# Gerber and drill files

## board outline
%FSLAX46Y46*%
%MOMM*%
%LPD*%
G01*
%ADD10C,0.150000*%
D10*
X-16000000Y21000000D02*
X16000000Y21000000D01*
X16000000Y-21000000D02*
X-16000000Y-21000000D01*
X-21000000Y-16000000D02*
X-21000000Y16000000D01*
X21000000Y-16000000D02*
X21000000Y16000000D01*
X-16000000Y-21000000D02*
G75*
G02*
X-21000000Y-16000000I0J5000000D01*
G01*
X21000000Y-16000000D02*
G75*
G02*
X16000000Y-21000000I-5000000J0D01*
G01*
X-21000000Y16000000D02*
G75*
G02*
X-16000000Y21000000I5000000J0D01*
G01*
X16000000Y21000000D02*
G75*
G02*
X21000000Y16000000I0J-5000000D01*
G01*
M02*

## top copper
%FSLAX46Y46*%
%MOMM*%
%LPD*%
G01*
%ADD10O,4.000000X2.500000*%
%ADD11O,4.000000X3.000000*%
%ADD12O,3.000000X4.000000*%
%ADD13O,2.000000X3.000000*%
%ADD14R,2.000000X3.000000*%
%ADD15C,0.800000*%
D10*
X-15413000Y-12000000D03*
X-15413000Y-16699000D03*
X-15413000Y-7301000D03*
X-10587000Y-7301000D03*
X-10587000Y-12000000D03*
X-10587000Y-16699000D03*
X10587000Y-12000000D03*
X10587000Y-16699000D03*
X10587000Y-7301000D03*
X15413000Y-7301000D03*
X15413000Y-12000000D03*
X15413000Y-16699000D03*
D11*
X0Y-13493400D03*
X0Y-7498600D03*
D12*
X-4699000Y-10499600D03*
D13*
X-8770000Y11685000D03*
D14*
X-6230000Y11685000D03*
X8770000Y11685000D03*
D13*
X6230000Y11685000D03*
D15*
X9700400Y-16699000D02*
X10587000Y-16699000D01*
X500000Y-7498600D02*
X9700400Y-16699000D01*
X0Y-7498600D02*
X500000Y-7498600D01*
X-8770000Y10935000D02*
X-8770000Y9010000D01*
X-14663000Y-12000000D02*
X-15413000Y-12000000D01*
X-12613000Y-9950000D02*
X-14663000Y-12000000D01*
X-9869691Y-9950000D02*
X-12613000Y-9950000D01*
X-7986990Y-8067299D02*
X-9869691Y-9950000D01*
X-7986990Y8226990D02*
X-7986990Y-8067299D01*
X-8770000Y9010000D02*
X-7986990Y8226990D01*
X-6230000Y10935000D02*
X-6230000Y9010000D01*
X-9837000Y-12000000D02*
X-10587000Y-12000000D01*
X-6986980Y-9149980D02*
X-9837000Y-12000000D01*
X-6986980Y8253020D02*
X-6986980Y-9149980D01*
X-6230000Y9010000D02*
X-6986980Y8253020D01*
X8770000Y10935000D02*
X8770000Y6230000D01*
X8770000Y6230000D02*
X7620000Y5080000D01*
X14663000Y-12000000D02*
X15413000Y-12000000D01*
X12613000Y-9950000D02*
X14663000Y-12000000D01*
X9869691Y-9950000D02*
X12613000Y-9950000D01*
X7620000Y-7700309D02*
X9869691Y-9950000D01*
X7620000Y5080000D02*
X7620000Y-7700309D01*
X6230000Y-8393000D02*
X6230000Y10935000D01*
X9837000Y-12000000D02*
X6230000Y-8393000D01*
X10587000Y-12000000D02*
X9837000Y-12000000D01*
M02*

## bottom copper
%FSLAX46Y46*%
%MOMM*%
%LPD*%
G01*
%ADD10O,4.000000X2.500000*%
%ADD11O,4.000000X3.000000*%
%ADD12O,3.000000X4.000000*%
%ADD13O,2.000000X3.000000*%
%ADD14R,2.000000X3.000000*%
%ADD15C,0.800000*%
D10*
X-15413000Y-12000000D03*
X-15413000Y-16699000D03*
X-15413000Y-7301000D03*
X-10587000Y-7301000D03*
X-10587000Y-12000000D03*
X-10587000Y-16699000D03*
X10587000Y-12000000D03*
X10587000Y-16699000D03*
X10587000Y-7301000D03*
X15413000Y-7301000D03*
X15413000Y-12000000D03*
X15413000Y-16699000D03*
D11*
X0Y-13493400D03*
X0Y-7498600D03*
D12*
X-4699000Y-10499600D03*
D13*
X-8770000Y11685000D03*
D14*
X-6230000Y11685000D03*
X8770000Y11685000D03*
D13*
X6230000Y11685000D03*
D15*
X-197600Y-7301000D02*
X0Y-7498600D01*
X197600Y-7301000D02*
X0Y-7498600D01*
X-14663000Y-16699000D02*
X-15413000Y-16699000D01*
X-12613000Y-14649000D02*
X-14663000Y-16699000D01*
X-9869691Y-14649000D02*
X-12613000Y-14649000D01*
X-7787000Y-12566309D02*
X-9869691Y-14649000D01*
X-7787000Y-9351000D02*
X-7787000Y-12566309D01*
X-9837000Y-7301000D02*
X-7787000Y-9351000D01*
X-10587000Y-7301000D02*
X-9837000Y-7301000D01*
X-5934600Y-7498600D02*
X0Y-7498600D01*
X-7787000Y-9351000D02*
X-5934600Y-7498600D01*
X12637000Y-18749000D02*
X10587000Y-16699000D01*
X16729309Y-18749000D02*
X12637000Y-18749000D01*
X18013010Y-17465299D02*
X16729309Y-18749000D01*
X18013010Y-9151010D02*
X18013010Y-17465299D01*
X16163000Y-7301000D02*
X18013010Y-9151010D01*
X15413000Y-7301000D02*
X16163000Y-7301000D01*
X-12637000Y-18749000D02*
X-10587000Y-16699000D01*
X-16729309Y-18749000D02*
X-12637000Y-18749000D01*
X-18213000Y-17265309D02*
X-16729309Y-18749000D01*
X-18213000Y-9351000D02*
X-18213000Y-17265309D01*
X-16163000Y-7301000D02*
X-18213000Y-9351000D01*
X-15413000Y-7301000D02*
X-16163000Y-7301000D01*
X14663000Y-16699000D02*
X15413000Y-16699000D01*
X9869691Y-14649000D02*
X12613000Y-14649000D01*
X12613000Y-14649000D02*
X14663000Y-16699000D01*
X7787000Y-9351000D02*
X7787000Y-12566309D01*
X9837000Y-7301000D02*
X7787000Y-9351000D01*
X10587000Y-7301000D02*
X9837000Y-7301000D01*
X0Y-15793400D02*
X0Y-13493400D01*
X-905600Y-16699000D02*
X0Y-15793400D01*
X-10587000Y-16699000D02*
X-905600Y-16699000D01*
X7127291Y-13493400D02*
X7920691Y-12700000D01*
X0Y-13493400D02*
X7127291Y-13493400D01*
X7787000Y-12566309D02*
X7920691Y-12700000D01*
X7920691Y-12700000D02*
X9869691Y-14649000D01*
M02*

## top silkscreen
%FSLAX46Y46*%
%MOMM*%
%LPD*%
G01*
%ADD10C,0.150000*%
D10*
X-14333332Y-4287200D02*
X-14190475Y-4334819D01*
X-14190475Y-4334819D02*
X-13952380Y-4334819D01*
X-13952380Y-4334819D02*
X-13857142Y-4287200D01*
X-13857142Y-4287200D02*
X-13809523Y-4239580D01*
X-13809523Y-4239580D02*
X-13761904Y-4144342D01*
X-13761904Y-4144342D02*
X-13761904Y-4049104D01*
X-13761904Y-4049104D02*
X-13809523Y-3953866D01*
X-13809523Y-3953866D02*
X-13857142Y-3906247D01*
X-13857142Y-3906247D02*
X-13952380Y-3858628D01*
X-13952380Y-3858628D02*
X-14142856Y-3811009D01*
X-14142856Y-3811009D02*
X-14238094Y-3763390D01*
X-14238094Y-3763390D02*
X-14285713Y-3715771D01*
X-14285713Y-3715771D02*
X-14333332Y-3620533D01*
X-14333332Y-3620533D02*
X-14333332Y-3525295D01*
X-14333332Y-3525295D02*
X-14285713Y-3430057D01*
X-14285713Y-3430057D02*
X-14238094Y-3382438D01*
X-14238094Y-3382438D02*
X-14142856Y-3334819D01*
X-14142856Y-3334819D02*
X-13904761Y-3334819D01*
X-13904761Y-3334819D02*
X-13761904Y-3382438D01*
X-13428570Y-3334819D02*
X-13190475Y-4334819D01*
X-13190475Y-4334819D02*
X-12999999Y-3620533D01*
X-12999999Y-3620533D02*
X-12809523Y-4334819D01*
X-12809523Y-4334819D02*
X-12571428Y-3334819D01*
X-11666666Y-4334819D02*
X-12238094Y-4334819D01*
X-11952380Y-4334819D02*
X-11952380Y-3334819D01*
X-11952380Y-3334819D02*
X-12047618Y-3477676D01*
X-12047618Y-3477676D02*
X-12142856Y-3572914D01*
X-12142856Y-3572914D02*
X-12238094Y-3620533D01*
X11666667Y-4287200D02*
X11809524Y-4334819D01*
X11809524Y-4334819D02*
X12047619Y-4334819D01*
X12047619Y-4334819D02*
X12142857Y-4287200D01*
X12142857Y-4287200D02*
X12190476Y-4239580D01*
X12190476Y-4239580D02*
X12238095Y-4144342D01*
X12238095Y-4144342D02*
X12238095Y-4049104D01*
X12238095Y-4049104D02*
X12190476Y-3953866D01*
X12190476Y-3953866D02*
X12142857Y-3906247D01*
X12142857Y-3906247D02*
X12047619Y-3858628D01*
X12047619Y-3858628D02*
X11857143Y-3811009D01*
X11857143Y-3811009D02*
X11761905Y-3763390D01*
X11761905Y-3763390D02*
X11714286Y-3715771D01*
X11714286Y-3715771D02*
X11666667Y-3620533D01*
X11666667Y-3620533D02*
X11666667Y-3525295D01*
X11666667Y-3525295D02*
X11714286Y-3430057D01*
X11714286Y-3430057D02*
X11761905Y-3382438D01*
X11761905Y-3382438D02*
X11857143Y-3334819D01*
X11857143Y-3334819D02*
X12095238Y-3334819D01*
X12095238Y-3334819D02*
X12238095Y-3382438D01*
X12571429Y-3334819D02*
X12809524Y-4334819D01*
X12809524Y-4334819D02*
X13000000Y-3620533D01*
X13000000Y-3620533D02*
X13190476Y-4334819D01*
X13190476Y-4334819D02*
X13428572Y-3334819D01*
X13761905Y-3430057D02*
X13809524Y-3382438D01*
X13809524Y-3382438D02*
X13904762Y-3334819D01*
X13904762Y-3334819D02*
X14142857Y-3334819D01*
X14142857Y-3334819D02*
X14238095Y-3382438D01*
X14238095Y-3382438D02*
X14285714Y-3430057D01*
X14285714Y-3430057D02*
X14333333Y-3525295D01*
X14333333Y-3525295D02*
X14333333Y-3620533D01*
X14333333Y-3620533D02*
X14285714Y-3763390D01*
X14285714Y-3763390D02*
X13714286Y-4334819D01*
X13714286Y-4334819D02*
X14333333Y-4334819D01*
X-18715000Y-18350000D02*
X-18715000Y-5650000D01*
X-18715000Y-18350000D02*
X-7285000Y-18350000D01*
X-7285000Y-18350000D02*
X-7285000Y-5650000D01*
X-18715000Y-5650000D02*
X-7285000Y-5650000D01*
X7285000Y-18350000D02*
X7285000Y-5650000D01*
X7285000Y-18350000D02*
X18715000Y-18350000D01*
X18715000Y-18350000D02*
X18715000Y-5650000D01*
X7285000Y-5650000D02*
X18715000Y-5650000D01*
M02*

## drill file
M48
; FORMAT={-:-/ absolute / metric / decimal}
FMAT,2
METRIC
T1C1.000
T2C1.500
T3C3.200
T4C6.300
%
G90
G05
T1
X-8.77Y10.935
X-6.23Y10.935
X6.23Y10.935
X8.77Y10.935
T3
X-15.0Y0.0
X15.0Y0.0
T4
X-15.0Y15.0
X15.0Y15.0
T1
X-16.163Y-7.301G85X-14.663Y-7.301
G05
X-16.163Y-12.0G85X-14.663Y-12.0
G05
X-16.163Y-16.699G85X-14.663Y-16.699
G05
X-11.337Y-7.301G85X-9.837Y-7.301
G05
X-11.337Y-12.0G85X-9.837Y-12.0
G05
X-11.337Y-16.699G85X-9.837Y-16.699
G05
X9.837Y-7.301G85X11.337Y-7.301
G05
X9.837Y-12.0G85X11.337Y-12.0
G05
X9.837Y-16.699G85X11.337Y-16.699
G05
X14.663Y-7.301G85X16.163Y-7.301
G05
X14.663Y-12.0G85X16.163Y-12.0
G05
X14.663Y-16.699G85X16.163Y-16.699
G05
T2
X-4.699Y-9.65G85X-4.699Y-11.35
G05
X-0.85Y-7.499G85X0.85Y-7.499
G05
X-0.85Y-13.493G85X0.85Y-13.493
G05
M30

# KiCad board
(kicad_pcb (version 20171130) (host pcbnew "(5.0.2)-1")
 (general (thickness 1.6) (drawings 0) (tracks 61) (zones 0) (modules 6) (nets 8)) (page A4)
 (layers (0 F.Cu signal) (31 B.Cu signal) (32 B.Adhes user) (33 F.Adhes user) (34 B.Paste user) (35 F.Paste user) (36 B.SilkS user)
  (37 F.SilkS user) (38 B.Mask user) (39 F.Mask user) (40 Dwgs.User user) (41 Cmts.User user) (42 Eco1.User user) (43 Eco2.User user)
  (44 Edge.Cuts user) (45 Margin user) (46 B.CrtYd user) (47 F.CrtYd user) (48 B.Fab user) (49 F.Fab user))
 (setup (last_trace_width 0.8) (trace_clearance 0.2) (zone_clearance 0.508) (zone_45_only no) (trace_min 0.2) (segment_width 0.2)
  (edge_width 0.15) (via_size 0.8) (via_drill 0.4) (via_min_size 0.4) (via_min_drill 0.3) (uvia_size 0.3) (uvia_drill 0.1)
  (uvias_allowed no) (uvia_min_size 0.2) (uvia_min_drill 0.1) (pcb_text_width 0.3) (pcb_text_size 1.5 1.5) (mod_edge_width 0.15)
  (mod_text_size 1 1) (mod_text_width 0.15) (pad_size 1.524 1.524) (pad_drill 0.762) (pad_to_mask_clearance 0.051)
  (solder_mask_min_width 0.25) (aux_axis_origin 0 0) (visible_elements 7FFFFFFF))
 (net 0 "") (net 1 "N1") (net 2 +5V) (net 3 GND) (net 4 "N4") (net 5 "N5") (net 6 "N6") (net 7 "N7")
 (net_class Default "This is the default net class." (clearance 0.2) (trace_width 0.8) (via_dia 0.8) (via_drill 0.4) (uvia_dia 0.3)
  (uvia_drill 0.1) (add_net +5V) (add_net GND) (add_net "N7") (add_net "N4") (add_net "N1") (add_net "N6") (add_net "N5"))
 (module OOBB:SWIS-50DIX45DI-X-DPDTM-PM (layer F.Cu) (at -15.413 7.301)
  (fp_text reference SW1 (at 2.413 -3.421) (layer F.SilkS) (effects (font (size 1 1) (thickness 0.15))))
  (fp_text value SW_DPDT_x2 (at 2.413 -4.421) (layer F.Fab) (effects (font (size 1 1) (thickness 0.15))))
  (fp_line (start -3.302 11.049) (end -3.302 -1.651) (layer F.SilkS) (width 0.15))
  (fp_line (start -3.302 11.049) (end 8.128 11.049) (layer F.SilkS) (width 0.15))
  (fp_line (start 8.128 11.049) (end 8.128 -1.651) (layer F.SilkS) (width 0.15))
  (fp_line (start -3.302 -1.651) (end 8.128 -1.651) (layer F.SilkS) (width 0.15))
  (pad 2 thru_hole oval (at 0 4.699) (size 4 2.5) (drill oval 2.5 1) (layers *.Cu *.Mask) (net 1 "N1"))
  (pad 1 thru_hole oval (at 0 9.398) (size 4 2.5) (drill oval 2.5 1) (layers *.Cu *.Mask) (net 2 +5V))
  (pad 3 thru_hole oval (at 0 0) (size 4 2.5) (drill oval 2.5 1) (layers *.Cu *.Mask) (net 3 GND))
  (pad 6 thru_hole oval (at 4.826 0) (size 4 2.5) (drill oval 2.5 1) (layers *.Cu *.Mask Eco1.User Eco2.User) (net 2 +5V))
  (pad 5 thru_hole oval (at 4.826 4.699) (size 4 2.5) (drill oval 2.5 1) (layers *.Cu *.Mask) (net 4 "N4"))
  (pad 4 thru_hole oval (at 4.826 9.398) (size 4 2.5) (drill oval 2.5 1) (layers *.Cu *.Mask) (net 3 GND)))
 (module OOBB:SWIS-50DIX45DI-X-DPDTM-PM (layer F.Cu) (at 10.587 7.301)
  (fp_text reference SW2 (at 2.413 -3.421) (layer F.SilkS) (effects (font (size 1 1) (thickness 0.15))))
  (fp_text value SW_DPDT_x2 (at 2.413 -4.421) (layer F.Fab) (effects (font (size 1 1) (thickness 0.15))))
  (fp_line (start -3.302 11.049) (end -3.302 -1.651) (layer F.SilkS) (width 0.15))
  (fp_line (start -3.302 11.049) (end 8.128 11.049) (layer F.SilkS) (width 0.15))
  (fp_line (start 8.128 11.049) (end 8.128 -1.651) (layer F.SilkS) (width 0.15))
  (fp_line (start -3.302 -1.651) (end 8.128 -1.651) (layer F.SilkS) (width 0.15))
  (pad 2 thru_hole oval (at 0 4.699) (size 4 2.5) (drill oval 2.5 1) (layers *.Cu *.Mask) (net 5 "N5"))
  (pad 1 thru_hole oval (at 0 9.398) (size 4 2.5) (drill oval 2.5 1) (layers *.Cu *.Mask) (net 2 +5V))
  (pad 3 thru_hole oval (at 0 0) (size 4 2.5) (drill oval 2.5 1) (layers *.Cu *.Mask) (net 3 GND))
  (pad 6 thru_hole oval (at 4.826 0) (size 4 2.5) (drill oval 2.5 1) (layers *.Cu *.Mask Eco1.User Eco2.User) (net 2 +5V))
  (pad 5 thru_hole oval (at 4.826 4.699) (size 4 2.5) (drill oval 2.5 1) (layers *.Cu *.Mask) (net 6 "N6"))
  (pad 4 thru_hole oval (at 4.826 9.398) (size 4 2.5) (drill oval 2.5 1) (layers *.Cu *.Mask) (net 3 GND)))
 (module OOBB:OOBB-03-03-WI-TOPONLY (layer F.Cu) (at 0 0)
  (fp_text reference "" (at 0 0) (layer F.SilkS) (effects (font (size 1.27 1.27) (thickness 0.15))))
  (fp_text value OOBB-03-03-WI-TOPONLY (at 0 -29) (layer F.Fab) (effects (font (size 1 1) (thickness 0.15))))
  (fp_line (start -16 -21) (end 16 -21) (layer Edge.Cuts) (width 0.15))
  (fp_line (start 16 21) (end -16 21) (layer Edge.Cuts) (width 0.15))
  (fp_line (start -21 16) (end -21 -16) (layer Edge.Cuts) (width 0.15))
  (fp_line (start 21 16) (end 21 -16) (layer Edge.Cuts) (width 0.15))
  (fp_arc (start -16 16) (end -16 21) (angle 90) (layer Edge.Cuts) (width 0.15))
  (fp_arc (start 16 16) (end 16 21) (angle -90) (layer Edge.Cuts) (width 0.15))
  (fp_arc (start -16 -16) (end -16 -21) (angle -90) (layer Edge.Cuts) (width 0.15))
  (fp_arc (start 16 -16) (end 16 -21) (angle 90) (layer Edge.Cuts) (width 0.15))
  (pad "" np_thru_hole circle (at 15 0) (size 3.2 3.2) (drill 3.2) (layers *.Cu *.Mask))
  (pad "" np_thru_hole circle (at 15 -15) (size 6.3 6.3) (drill 6.3) (layers *.Cu *.Mask))
  (pad "" np_thru_hole circle (at -15 0) (size 3.2 3.2) (drill 3.2) (layers *.Cu *.Mask))
  (pad "" np_thru_hole circle (at -15 -15) (size 6.3 6.3) (drill 6.3) (layers *.Cu *.Mask)))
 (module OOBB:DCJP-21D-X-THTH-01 (layer B.Cu) (at 0 13.7 90)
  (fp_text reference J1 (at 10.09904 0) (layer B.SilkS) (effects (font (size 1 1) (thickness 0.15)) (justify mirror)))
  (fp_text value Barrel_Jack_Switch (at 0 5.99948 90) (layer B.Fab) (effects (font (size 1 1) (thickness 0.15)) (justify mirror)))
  (pad 2 thru_hole oval (at 0.2066 0 90) (size 3 4) (drill oval 1.5 3.2) (layers *.Cu *.Mask) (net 3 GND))
  (pad 1 thru_hole oval (at 6.2014 0 90) (size 3 4) (drill oval 1.5 3.2) (layers *.Cu *.Mask) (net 2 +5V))
  (pad 3 thru_hole oval (at 3.2004 -4.699) (size 3 4) (drill oval 1.5 3.2) (layers *.Cu *.Mask) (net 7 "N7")))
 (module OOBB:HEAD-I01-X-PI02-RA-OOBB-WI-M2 (layer B.Cu) (at -6.23 -10.935 90)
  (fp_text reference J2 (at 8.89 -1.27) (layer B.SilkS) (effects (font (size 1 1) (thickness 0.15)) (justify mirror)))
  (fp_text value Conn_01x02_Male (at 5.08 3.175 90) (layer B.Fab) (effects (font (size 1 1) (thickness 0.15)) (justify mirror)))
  (pad 2 thru_hole oval (at 0 -2.54 90) (size 3 2) (drill 1 (offset 0.75 0)) (layers *.Cu *.Mask) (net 1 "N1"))
  (pad 1 thru_hole rect (at 0 0 90) (size 3 2) (drill 1 (offset 0.75 0)) (layers *.Cu *.Mask) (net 4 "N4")))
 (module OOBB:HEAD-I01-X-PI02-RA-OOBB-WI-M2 (layer B.Cu) (at 8.77 -10.935 90)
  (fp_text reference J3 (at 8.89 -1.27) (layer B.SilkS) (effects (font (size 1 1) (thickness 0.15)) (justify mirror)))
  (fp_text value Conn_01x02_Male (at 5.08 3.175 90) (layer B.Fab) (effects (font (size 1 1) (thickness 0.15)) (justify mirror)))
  (pad 1 thru_hole rect (at 0 0 90) (size 3 2) (drill 1 (offset 0.75 0)) (layers *.Cu *.Mask) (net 6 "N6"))
  (pad 2 thru_hole oval (at 0 -2.54 90) (size 3 2) (drill 1 (offset 0.75 0)) (layers *.Cu *.Mask) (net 5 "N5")))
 (segment (start -0.1976 7.301) (end 0 7.4986) (width 0.8) (layer B.Cu) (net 2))
 (segment (start 0.1976 7.301) (end 0 7.4986) (width 0.8) (layer B.Cu) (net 2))
 (segment (start -14.663 16.699) (end -15.413 16.699) (width 0.8) (layer B.Cu) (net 2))
 (segment (start -12.613 14.649) (end -14.663 16.699) (width 0.8) (layer B.Cu) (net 2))
 (segment (start -9.869691 14.649) (end -12.613 14.649) (width 0.8) (layer B.Cu) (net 2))
 (segment (start -7.787 12.566309) (end -9.869691 14.649) (width 0.8) (layer B.Cu) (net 2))
 (segment (start -7.787 9.351) (end -7.787 12.566309) (width 0.8) (layer B.Cu) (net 2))
 (segment (start -9.837 7.301) (end -7.787 9.351) (width 0.8) (layer B.Cu) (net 2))
 (segment (start -10.587 7.301) (end -9.837 7.301) (width 0.8) (layer B.Cu) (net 2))
 (segment (start -5.9346 7.4986) (end 0 7.4986) (width 0.8) (layer B.Cu) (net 2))
 (segment (start -7.787 9.351) (end -5.9346 7.4986) (width 0.8) (layer B.Cu) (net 2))
 (segment (start 12.637 18.749) (end 10.587 16.699) (width 0.8) (layer B.Cu) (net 2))
 (segment (start 16.729309 18.749) (end 12.637 18.749) (width 0.8) (layer B.Cu) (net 2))
 (segment (start 18.01301 17.465299) (end 16.729309 18.749) (width 0.8) (layer B.Cu) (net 2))
 (segment (start 18.01301 9.15101) (end 18.01301 17.465299) (width 0.8) (layer B.Cu) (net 2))
 (segment (start 16.163 7.301) (end 18.01301 9.15101) (width 0.8) (layer B.Cu) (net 2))
 (segment (start 15.413 7.301) (end 16.163 7.301) (width 0.8) (layer B.Cu) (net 2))
 (segment (start 9.7004 16.699) (end 10.587 16.699) (width 0.8) (layer F.Cu) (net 2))
 (segment (start 0.5 7.4986) (end 9.7004 16.699) (width 0.8) (layer F.Cu) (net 2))
 (segment (start 0 7.4986) (end 0.5 7.4986) (width 0.8) (layer F.Cu) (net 2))
 (segment (start -12.637 18.749) (end -10.587 16.699) (width 0.8) (layer B.Cu) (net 3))
 (segment (start -16.729309 18.749) (end -12.637 18.749) (width 0.8) (layer B.Cu) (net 3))
 (segment (start -18.213 17.265309) (end -16.729309 18.749) (width 0.8) (layer B.Cu) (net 3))
 (segment (start -18.213 9.351) (end -18.213 17.265309) (width 0.8) (layer B.Cu) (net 3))
 (segment (start -16.163 7.301) (end -18.213 9.351) (width 0.8) (layer B.Cu) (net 3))
 (segment (start -15.413 7.301) (end -16.163 7.301) (width 0.8) (layer B.Cu) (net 3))
 (segment (start 14.663 16.699) (end 15.413 16.699) (width 0.8) (layer B.Cu) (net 3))
 (segment (start 9.869691 14.649) (end 12.613 14.649) (width 0.8) (layer B.Cu) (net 3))
 (segment (start 12.613 14.649) (end 14.663 16.699) (width 0.8) (layer B.Cu) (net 3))
 (segment (start 7.787 9.351) (end 7.787 12.566309) (width 0.8) (layer B.Cu) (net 3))
 (segment (start 9.837 7.301) (end 7.787 9.351) (width 0.8) (layer B.Cu) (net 3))
 (segment (start 10.587 7.301) (end 9.837 7.301) (width 0.8) (layer B.Cu) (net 3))
 (segment (start 0 15.7934) (end 0 13.4934) (width 0.8) (layer B.Cu) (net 3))
 (segment (start -0.9056 16.699) (end 0 15.7934) (width 0.8) (layer B.Cu) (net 3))
 (segment (start -10.587 16.699) (end -0.9056 16.699) (width 0.8) (layer B.Cu) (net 3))
 (segment (start 7.127291 13.4934) (end 7.920691 12.7) (width 0.8) (layer B.Cu) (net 3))
 (segment (start 0 13.4934) (end 7.127291 13.4934) (width 0.8) (layer B.Cu) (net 3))
 (segment (start 7.787 12.566309) (end 7.920691 12.7) (width 0.8) (layer B.Cu) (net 3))
 (segment (start 7.920691 12.7) (end 9.869691 14.649) (width 0.8) (layer B.Cu) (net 3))
 (segment (start -8.77 -10.935) (end -8.77 -9.01) (width 0.8) (layer F.Cu) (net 1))
 (segment (start -14.663 12) (end -15.413 12) (width 0.8) (layer F.Cu) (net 1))
 (segment (start -12.613 9.95) (end -14.663 12) (width 0.8) (layer F.Cu) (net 1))
 (segment (start -9.869691 9.95) (end -12.613 9.95) (width 0.8) (layer F.Cu) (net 1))
 (segment (start -7.98699 8.067299) (end -9.869691 9.95) (width 0.8) (layer F.Cu) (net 1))
 (segment (start -7.98699 -8.22699) (end -7.98699 8.067299) (width 0.8) (layer F.Cu) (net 1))
 (segment (start -8.77 -9.01) (end -7.98699 -8.22699) (width 0.8) (layer F.Cu) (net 1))
 (segment (start -6.23 -10.935) (end -6.23 -9.01) (width 0.8) (layer F.Cu) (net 4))
 (segment (start -9.837 12) (end -10.587 12) (width 0.8) (layer F.Cu) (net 4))
 (segment (start -6.98698 9.14998) (end -9.837 12) (width 0.8) (layer F.Cu) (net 4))
 (segment (start -6.98698 -8.25302) (end -6.98698 9.14998) (width 0.8) (layer F.Cu) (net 4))
 (segment (start -6.23 -9.01) (end -6.98698 -8.25302) (width 0.8) (layer F.Cu) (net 4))
 (segment (start 8.77 -10.935) (end 8.77 -6.23) (width 0.8) (layer F.Cu) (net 6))
 (segment (start 8.77 -6.23) (end 7.62 -5.08) (width 0.8) (layer F.Cu) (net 6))
 (segment (start 14.663 12) (end 15.413 12) (width 0.8) (layer F.Cu) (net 6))
 (segment (start 12.613 9.95) (end 14.663 12) (width 0.8) (layer F.Cu) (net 6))
 (segment (start 9.869691 9.95) (end 12.613 9.95) (width 0.8) (layer F.Cu) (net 6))
 (segment (start 7.62 7.700309) (end 9.869691 9.95) (width 0.8) (layer F.Cu) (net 6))
 (segment (start 7.62 -5.08) (end 7.62 7.700309) (width 0.8) (layer F.Cu) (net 6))
 (segment (start 6.23 8.393) (end 6.23 -10.935) (width 0.8) (layer F.Cu) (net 5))
 (segment (start 9.837 12) (end 6.23 8.393) (width 0.8) (layer F.Cu) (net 5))
 (segment (start 10.587 12) (end 9.837 12) (width 0.8) (layer F.Cu) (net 5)))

